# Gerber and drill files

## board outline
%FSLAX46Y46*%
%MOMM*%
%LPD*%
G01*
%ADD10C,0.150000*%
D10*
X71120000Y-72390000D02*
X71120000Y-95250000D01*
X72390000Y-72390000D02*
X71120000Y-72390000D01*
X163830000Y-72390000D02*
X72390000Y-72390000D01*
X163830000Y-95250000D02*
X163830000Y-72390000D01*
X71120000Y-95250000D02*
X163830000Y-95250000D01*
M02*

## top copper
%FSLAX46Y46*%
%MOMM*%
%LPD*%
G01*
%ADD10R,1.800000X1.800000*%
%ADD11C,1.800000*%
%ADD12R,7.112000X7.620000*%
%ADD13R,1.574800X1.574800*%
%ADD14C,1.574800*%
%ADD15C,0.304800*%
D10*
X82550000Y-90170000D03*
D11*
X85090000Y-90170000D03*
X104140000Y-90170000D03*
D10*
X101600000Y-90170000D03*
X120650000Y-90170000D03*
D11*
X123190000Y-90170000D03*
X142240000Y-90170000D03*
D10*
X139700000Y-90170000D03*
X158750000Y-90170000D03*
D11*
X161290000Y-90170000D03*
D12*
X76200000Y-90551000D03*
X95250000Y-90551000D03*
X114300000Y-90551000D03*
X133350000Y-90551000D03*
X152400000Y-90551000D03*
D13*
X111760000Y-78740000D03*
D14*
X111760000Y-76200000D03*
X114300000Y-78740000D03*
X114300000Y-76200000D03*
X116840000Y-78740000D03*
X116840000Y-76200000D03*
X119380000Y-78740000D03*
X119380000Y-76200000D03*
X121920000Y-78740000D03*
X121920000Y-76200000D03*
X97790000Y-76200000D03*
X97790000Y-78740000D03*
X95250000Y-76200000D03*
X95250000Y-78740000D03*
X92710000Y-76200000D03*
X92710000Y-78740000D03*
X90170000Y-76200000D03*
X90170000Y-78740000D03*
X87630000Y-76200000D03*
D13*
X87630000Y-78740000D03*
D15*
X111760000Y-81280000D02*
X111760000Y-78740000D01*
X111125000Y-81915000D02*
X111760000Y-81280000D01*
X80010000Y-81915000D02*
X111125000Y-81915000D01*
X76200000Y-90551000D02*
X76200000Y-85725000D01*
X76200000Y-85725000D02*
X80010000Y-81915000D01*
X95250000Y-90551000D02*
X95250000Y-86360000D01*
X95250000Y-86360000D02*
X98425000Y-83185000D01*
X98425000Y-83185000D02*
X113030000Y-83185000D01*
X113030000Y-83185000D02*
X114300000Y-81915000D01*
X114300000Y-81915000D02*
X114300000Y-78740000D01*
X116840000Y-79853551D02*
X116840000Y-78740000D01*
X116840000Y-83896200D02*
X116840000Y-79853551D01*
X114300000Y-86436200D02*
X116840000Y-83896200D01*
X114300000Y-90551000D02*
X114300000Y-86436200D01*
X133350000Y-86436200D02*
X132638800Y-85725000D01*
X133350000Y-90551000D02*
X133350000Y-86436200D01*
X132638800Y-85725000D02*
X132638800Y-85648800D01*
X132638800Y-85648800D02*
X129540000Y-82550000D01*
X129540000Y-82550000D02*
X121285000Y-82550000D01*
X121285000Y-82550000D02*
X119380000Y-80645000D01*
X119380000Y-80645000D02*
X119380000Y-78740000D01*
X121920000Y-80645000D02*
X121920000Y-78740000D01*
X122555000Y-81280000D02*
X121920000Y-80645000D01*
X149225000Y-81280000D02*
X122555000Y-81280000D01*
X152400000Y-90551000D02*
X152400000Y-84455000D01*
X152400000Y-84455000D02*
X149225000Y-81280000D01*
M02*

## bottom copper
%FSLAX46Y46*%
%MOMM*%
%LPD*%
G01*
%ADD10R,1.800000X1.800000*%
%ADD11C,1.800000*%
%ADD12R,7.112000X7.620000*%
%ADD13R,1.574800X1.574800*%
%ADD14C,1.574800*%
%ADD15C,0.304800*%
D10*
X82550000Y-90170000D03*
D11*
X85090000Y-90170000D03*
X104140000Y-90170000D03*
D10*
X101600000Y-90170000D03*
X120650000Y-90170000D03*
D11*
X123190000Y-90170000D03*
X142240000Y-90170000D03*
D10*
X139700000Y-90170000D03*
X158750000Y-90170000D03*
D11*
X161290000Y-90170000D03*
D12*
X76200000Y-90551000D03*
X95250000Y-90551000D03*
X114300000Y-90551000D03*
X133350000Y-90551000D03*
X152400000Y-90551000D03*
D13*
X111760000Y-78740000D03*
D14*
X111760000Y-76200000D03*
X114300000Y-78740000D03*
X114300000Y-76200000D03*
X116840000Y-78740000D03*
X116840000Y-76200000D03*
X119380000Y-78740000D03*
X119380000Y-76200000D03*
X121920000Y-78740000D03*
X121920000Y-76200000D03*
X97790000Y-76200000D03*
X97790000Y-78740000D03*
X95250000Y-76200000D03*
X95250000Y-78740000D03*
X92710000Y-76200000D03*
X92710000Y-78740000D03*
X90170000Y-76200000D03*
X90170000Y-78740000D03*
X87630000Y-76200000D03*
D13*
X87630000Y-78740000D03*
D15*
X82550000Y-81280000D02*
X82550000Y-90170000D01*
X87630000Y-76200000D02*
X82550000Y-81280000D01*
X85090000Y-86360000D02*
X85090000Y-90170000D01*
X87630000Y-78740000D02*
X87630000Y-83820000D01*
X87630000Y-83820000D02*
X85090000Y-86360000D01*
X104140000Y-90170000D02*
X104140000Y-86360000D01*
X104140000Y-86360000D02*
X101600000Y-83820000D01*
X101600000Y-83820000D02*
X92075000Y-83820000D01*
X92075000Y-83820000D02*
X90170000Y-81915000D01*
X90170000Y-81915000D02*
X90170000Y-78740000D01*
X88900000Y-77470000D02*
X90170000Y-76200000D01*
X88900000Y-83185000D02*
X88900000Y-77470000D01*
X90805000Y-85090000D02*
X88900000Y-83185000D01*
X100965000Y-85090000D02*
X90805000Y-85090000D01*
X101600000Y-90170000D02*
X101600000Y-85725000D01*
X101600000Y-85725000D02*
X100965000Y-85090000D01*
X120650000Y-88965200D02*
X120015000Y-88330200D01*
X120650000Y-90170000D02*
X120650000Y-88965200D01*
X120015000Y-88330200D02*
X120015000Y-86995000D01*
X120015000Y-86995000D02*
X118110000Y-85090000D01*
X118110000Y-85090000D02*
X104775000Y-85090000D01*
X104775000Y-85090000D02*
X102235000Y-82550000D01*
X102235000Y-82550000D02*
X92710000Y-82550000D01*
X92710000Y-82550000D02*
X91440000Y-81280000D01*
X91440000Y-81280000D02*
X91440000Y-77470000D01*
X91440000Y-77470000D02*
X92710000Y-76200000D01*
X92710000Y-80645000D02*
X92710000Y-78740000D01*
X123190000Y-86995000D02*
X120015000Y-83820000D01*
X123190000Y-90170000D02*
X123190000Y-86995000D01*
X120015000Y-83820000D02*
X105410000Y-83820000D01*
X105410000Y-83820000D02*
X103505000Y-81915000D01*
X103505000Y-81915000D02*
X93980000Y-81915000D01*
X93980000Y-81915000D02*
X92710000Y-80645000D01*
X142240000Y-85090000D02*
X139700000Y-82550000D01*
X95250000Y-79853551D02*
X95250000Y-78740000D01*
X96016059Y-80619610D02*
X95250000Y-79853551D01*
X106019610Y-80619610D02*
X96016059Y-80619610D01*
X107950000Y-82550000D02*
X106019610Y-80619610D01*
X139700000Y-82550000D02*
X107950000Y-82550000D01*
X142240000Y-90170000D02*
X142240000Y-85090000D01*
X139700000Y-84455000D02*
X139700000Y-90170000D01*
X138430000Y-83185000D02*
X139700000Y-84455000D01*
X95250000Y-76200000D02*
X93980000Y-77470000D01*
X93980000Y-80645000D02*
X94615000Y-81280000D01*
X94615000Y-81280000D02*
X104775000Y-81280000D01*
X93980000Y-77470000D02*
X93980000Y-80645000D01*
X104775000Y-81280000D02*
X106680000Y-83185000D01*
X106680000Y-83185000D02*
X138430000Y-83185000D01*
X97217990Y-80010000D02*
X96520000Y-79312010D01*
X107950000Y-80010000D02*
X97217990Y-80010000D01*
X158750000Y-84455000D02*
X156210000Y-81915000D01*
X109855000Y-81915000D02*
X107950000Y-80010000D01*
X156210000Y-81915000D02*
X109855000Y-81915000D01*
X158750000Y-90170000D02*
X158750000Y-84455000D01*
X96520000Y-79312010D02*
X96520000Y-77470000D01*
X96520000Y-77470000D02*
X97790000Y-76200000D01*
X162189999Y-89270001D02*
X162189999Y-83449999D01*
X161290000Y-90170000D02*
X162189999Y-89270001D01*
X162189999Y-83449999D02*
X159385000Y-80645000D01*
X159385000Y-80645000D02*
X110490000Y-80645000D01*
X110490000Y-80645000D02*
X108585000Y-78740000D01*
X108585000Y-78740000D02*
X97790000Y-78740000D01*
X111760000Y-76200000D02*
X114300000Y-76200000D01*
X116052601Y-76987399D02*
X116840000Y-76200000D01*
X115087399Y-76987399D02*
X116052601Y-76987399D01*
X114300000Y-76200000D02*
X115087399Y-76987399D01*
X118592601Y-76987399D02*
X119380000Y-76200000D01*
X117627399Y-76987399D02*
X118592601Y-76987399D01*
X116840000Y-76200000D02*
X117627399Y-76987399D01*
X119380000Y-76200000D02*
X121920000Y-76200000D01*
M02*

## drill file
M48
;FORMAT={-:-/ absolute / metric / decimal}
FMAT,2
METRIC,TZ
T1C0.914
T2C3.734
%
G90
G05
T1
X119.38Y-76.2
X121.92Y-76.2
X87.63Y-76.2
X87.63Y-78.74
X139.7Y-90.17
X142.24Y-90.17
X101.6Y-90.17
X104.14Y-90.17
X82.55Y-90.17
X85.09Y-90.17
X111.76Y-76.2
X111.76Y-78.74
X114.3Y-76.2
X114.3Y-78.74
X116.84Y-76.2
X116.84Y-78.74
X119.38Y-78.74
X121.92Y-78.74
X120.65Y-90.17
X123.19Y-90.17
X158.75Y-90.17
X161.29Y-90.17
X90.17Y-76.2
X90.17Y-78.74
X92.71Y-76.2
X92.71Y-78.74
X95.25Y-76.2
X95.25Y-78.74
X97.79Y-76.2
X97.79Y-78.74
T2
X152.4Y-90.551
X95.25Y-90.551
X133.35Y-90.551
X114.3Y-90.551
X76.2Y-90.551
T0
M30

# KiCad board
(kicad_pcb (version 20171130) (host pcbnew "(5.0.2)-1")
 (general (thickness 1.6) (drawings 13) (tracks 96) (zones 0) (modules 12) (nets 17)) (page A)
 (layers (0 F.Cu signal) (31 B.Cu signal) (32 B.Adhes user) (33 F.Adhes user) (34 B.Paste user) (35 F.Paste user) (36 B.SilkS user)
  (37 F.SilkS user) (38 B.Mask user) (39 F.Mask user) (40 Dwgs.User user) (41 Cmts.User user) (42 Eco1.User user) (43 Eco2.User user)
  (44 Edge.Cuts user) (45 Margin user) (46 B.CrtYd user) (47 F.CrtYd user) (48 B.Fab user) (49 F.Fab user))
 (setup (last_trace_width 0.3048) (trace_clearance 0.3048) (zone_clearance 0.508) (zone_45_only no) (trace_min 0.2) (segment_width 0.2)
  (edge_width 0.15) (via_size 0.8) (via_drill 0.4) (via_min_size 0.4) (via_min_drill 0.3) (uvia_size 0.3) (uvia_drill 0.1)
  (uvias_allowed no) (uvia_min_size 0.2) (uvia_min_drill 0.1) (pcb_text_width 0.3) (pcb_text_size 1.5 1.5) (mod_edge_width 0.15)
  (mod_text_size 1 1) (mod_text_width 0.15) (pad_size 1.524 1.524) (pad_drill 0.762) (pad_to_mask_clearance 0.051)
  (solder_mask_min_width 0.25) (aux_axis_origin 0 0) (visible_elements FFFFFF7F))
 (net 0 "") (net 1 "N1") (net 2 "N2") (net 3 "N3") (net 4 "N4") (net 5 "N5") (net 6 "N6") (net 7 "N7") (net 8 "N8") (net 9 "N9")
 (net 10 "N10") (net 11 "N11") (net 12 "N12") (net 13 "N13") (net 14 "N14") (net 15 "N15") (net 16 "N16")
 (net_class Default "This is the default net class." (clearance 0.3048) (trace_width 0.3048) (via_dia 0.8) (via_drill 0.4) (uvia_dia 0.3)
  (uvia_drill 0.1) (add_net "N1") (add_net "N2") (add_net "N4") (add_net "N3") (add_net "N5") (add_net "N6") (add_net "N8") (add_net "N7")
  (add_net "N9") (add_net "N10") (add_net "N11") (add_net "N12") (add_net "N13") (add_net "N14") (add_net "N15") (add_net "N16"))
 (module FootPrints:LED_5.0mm (layer F.Cu) (at 82.55 90.17)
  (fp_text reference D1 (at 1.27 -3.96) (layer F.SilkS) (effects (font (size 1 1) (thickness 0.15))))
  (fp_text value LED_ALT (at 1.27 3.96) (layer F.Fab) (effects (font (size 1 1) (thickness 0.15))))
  (pad 1 thru_hole rect (at 0 0) (size 1.8 1.8) (drill 0.9144) (layers *.Cu *.Mask) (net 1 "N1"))
  (pad 2 thru_hole circle (at 2.54 0) (size 1.8 1.8) (drill 0.9144) (layers *.Cu *.Mask) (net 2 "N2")))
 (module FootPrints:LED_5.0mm (layer F.Cu) (at 101.6 90.17)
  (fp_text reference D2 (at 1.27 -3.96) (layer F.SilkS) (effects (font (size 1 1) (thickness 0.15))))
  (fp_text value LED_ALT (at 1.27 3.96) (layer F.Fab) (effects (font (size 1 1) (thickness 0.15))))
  (pad 2 thru_hole circle (at 2.54 0) (size 1.8 1.8) (drill 0.9144) (layers *.Cu *.Mask) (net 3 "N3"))
  (pad 1 thru_hole rect (at 0 0) (size 1.8 1.8) (drill 0.9144) (layers *.Cu *.Mask) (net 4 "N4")))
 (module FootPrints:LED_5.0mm (layer F.Cu) (at 120.65 90.17)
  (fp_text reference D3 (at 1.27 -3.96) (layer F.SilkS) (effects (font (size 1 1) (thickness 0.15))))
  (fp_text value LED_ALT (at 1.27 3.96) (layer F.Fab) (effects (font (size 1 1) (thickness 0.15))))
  (pad 1 thru_hole rect (at 0 0) (size 1.8 1.8) (drill 0.9144) (layers *.Cu *.Mask) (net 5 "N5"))
  (pad 2 thru_hole circle (at 2.54 0) (size 1.8 1.8) (drill 0.9144) (layers *.Cu *.Mask) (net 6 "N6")))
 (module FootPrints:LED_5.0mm (layer F.Cu) (at 139.7 90.17)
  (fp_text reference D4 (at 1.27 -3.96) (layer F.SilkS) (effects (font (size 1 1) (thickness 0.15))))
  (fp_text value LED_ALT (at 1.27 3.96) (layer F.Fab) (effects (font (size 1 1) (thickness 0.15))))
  (pad 2 thru_hole circle (at 2.54 0) (size 1.8 1.8) (drill 0.9144) (layers *.Cu *.Mask) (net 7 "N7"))
  (pad 1 thru_hole rect (at 0 0) (size 1.8 1.8) (drill 0.9144) (layers *.Cu *.Mask) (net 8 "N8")))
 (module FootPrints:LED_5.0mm (layer F.Cu) (at 158.75 90.17)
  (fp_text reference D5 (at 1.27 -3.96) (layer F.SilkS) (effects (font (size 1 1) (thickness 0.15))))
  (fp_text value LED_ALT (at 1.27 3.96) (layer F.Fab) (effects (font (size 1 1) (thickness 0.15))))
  (pad 1 thru_hole rect (at 0 0) (size 1.8 1.8) (drill 0.9144) (layers *.Cu *.Mask) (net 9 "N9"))
  (pad 2 thru_hole circle (at 2.54 0) (size 1.8 1.8) (drill 0.9144) (layers *.Cu *.Mask) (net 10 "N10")))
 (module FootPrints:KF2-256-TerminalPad (layer F.Cu) (at 76.2 95.25)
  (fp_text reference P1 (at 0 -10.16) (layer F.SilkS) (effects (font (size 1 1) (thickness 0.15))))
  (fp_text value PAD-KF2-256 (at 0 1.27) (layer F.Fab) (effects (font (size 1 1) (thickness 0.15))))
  (pad 1 thru_hole rect (at 0 -4.699) (size 7.112 7.62) (drill 3.7338) (layers *.Cu *.Mask F.SilkS) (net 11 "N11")))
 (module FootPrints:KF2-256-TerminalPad (layer F.Cu) (at 95.25 95.25)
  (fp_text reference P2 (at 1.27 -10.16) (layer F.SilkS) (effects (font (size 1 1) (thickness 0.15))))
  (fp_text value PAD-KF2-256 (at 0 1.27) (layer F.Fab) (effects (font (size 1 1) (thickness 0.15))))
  (pad 1 thru_hole rect (at 0 -4.699) (size 7.112 7.62) (drill 3.7338) (layers *.Cu *.Mask F.SilkS) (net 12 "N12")))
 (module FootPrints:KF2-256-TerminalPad (layer F.Cu) (at 114.3 95.25)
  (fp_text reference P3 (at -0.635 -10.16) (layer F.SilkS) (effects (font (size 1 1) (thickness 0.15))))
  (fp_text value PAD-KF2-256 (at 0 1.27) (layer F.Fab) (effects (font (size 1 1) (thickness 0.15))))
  (pad 1 thru_hole rect (at 0 -4.699) (size 7.112 7.62) (drill 3.7338) (layers *.Cu *.Mask F.SilkS) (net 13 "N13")))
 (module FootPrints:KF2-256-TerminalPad (layer F.Cu) (at 133.35 95.25)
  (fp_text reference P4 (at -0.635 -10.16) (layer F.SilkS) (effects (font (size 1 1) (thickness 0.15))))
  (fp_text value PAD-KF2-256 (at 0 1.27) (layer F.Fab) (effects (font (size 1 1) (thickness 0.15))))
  (pad 1 thru_hole rect (at 0 -4.699) (size 7.112 7.62) (drill 3.7338) (layers *.Cu *.Mask F.SilkS) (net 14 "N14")))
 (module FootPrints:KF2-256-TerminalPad (layer F.Cu) (at 152.4 95.25)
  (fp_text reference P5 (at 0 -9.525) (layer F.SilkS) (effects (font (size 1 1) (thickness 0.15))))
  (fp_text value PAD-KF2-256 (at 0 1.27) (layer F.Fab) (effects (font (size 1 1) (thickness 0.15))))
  (pad 1 thru_hole rect (at 0 -4.699) (size 7.112 7.62) (drill 3.7338) (layers *.Cu *.Mask F.SilkS) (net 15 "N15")))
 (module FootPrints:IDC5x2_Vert (layer F.Cu) (at 116.84 77.47 180)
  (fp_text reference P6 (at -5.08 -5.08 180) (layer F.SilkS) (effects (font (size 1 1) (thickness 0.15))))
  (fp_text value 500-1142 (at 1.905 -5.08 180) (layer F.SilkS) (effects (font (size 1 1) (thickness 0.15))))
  (pad 1 thru_hole rect (at 5.08 -1.27 180) (size 1.5748 1.5748) (drill 0.9144) (layers *.Cu *.Mask F.SilkS) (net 11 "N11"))
  (pad 2 thru_hole circle (at 5.08 1.27 180) (size 1.5748 1.5748) (drill 0.9144) (layers *.Cu *.Mask F.SilkS) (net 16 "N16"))
  (pad 3 thru_hole circle (at 2.54 -1.27 180) (size 1.5748 1.5748) (drill 0.9144) (layers *.Cu *.Mask F.SilkS) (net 12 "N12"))
  (pad 4 thru_hole circle (at 2.54 1.27 180) (size 1.5748 1.5748) (drill 0.9144) (layers *.Cu *.Mask F.SilkS) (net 16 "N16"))
  (pad 5 thru_hole circle (at 0 -1.27 180) (size 1.5748 1.5748) (drill 0.9144) (layers *.Cu *.Mask F.SilkS) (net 13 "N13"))
  (pad 6 thru_hole circle (at 0 1.27 180) (size 1.5748 1.5748) (drill 0.9144) (layers *.Cu *.Mask F.SilkS) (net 16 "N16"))
  (pad 7 thru_hole circle (at -2.54 -1.27 180) (size 1.5748 1.5748) (drill 0.9144) (layers *.Cu *.Mask F.SilkS) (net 14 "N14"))
  (pad 8 thru_hole circle (at -2.54 1.27 180) (size 1.5748 1.5748) (drill 0.9144) (layers *.Cu *.Mask F.SilkS) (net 16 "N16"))
  (pad 9 thru_hole circle (at -5.08 -1.27 180) (size 1.5748 1.5748) (drill 0.9144) (layers *.Cu *.Mask F.SilkS) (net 15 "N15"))
  (pad 10 thru_hole circle (at -5.08 1.27 180) (size 1.5748 1.5748) (drill 0.9144) (layers *.Cu *.Mask F.SilkS) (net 16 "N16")))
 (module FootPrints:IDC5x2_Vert (layer F.Cu) (at 92.71 77.47 180)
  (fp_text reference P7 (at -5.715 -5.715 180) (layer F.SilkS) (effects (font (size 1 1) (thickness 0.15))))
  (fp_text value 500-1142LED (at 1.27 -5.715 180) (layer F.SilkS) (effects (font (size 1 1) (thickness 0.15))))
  (pad 10 thru_hole circle (at -5.08 1.27 180) (size 1.5748 1.5748) (drill 0.9144) (layers *.Cu *.Mask F.SilkS) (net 9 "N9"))
  (pad 9 thru_hole circle (at -5.08 -1.27 180) (size 1.5748 1.5748) (drill 0.9144) (layers *.Cu *.Mask F.SilkS) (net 10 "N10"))
  (pad 8 thru_hole circle (at -2.54 1.27 180) (size 1.5748 1.5748) (drill 0.9144) (layers *.Cu *.Mask F.SilkS) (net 8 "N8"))
  (pad 7 thru_hole circle (at -2.54 -1.27 180) (size 1.5748 1.5748) (drill 0.9144) (layers *.Cu *.Mask F.SilkS) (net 7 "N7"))
  (pad 6 thru_hole circle (at 0 1.27 180) (size 1.5748 1.5748) (drill 0.9144) (layers *.Cu *.Mask F.SilkS) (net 5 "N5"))
  (pad 5 thru_hole circle (at 0 -1.27 180) (size 1.5748 1.5748) (drill 0.9144) (layers *.Cu *.Mask F.SilkS) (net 6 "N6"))
  (pad 4 thru_hole circle (at 2.54 1.27 180) (size 1.5748 1.5748) (drill 0.9144) (layers *.Cu *.Mask F.SilkS) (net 4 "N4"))
  (pad 3 thru_hole circle (at 2.54 -1.27 180) (size 1.5748 1.5748) (drill 0.9144) (layers *.Cu *.Mask F.SilkS) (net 3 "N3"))
  (pad 2 thru_hole circle (at 5.08 1.27 180) (size 1.5748 1.5748) (drill 0.9144) (layers *.Cu *.Mask F.SilkS) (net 1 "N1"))
  (pad 1 thru_hole rect (at 5.08 -1.27 180) (size 1.5748 1.5748) (drill 0.9144) (layers *.Cu *.Mask F.SilkS) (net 2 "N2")))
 (gr_line (start 71.12 72.39) (end 71.12 95.25) (layer Edge.Cuts) (width 0.15))
 (gr_line (start 72.39 72.39) (end 71.12 72.39) (layer Edge.Cuts) (width 0.15))
 (gr_line (start 163.83 72.39) (end 72.39 72.39) (layer Edge.Cuts) (width 0.15))
 (gr_line (start 163.83 95.25) (end 163.83 72.39) (layer Edge.Cuts) (width 0.15))
 (gr_line (start 71.12 95.25) (end 163.83 95.25) (layer Edge.Cuts) (width 0.15))
 (segment (start 82.55 81.28) (end 82.55 90.17) (width 0.3048) (layer B.Cu) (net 1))
 (segment (start 87.63 76.2) (end 82.55 81.28) (width 0.3048) (layer B.Cu) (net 1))
 (segment (start 85.09 86.36) (end 85.09 90.17) (width 0.3048) (layer B.Cu) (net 2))
 (segment (start 87.63 78.74) (end 87.63 83.82) (width 0.3048) (layer B.Cu) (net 2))
 (segment (start 87.63 83.82) (end 85.09 86.36) (width 0.3048) (layer B.Cu) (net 2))
 (segment (start 104.14 90.17) (end 104.14 86.36) (width 0.3048) (layer B.Cu) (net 3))
 (segment (start 104.14 86.36) (end 101.6 83.82) (width 0.3048) (layer B.Cu) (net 3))
 (segment (start 101.6 83.82) (end 92.075 83.82) (width 0.3048) (layer B.Cu) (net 3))
 (segment (start 92.075 83.82) (end 90.17 81.915) (width 0.3048) (layer B.Cu) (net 3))
 (segment (start 90.17 81.915) (end 90.17 78.74) (width 0.3048) (layer B.Cu) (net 3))
 (segment (start 88.9 77.47) (end 90.17 76.2) (width 0.3048) (layer B.Cu) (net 4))
 (segment (start 88.9 83.185) (end 88.9 77.47) (width 0.3048) (layer B.Cu) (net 4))
 (segment (start 90.805 85.09) (end 88.9 83.185) (width 0.3048) (layer B.Cu) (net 4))
 (segment (start 100.965 85.09) (end 90.805 85.09) (width 0.3048) (layer B.Cu) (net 4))
 (segment (start 101.6 90.17) (end 101.6 85.725) (width 0.3048) (layer B.Cu) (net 4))
 (segment (start 101.6 85.725) (end 100.965 85.09) (width 0.3048) (layer B.Cu) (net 4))
 (segment (start 120.65 88.9652) (end 120.015 88.3302) (width 0.3048) (layer B.Cu) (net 5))
 (segment (start 120.65 90.17) (end 120.65 88.9652) (width 0.3048) (layer B.Cu) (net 5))
 (segment (start 120.015 88.3302) (end 120.015 86.995) (width 0.3048) (layer B.Cu) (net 5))
 (segment (start 120.015 86.995) (end 118.11 85.09) (width 0.3048) (layer B.Cu) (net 5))
 (segment (start 118.11 85.09) (end 104.775 85.09) (width 0.3048) (layer B.Cu) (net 5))
 (segment (start 104.775 85.09) (end 102.235 82.55) (width 0.3048) (layer B.Cu) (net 5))
 (segment (start 102.235 82.55) (end 92.71 82.55) (width 0.3048) (layer B.Cu) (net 5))
 (segment (start 92.71 82.55) (end 91.44 81.28) (width 0.3048) (layer B.Cu) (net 5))
 (segment (start 91.44 81.28) (end 91.44 77.47) (width 0.3048) (layer B.Cu) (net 5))
 (segment (start 91.44 77.47) (end 92.71 76.2) (width 0.3048) (layer B.Cu) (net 5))
 (segment (start 92.71 80.645) (end 92.71 78.74) (width 0.3048) (layer B.Cu) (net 6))
 (segment (start 123.19 86.995) (end 120.015 83.82) (width 0.3048) (layer B.Cu) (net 6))
 (segment (start 123.19 90.17) (end 123.19 86.995) (width 0.3048) (layer B.Cu) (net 6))
 (segment (start 120.015 83.82) (end 105.41 83.82) (width 0.3048) (layer B.Cu) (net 6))
 (segment (start 105.41 83.82) (end 103.505 81.915) (width 0.3048) (layer B.Cu) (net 6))
 (segment (start 103.505 81.915) (end 93.98 81.915) (width 0.3048) (layer B.Cu) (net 6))
 (segment (start 93.98 81.915) (end 92.71 80.645) (width 0.3048) (layer B.Cu) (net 6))
 (segment (start 142.24 85.09) (end 139.7 82.55) (width 0.3048) (layer B.Cu) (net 7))
 (segment (start 95.25 79.853551) (end 95.25 78.74) (width 0.3048) (layer B.Cu) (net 7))
 (segment (start 96.016059 80.61961) (end 95.25 79.853551) (width 0.3048) (layer B.Cu) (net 7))
 (segment (start 106.01961 80.61961) (end 96.016059 80.61961) (width 0.3048) (layer B.Cu) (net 7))
 (segment (start 107.95 82.55) (end 106.01961 80.61961) (width 0.3048) (layer B.Cu) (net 7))
 (segment (start 139.7 82.55) (end 107.95 82.55) (width 0.3048) (layer B.Cu) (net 7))
 (segment (start 142.24 90.17) (end 142.24 85.09) (width 0.3048) (layer B.Cu) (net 7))
 (segment (start 139.7 84.455) (end 139.7 90.17) (width 0.3048) (layer B.Cu) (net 8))
 (segment (start 138.43 83.185) (end 139.7 84.455) (width 0.3048) (layer B.Cu) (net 8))
 (segment (start 95.25 76.2) (end 93.98 77.47) (width 0.3048) (layer B.Cu) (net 8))
 (segment (start 93.98 80.645) (end 94.615 81.28) (width 0.3048) (layer B.Cu) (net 8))
 (segment (start 94.615 81.28) (end 104.775 81.28) (width 0.3048) (layer B.Cu) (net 8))
 (segment (start 93.98 77.47) (end 93.98 80.645) (width 0.3048) (layer B.Cu) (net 8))
 (segment (start 104.775 81.28) (end 106.68 83.185) (width 0.3048) (layer B.Cu) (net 8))
 (segment (start 106.68 83.185) (end 138.43 83.185) (width 0.3048) (layer B.Cu) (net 8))
 (segment (start 97.21799 80.01) (end 96.52 79.31201) (width 0.3048) (layer B.Cu) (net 9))
 (segment (start 107.95 80.01) (end 97.21799 80.01) (width 0.3048) (layer B.Cu) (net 9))
 (segment (start 158.75 84.455) (end 156.21 81.915) (width 0.3048) (layer B.Cu) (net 9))
 (segment (start 109.855 81.915) (end 107.95 80.01) (width 0.3048) (layer B.Cu) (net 9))
 (segment (start 156.21 81.915) (end 109.855 81.915) (width 0.3048) (layer B.Cu) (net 9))
 (segment (start 158.75 90.17) (end 158.75 84.455) (width 0.3048) (layer B.Cu) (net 9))
 (segment (start 96.52 79.31201) (end 96.52 77.47) (width 0.3048) (layer B.Cu) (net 9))
 (segment (start 96.52 77.47) (end 97.79 76.2) (width 0.3048) (layer B.Cu) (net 9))
 (segment (start 162.189999 89.270001) (end 162.189999 83.449999) (width 0.3048) (layer B.Cu) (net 10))
 (segment (start 161.29 90.17) (end 162.189999 89.270001) (width 0.3048) (layer B.Cu) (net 10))
 (segment (start 162.189999 83.449999) (end 159.385 80.645) (width 0.3048) (layer B.Cu) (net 10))
 (segment (start 159.385 80.645) (end 110.49 80.645) (width 0.3048) (layer B.Cu) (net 10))
 (segment (start 110.49 80.645) (end 108.585 78.74) (width 0.3048) (layer B.Cu) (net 10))
 (segment (start 108.585 78.74) (end 97.79 78.74) (width 0.3048) (layer B.Cu) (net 10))
 (segment (start 111.76 81.28) (end 111.76 78.74) (width 0.3048) (layer F.Cu) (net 11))
 (segment (start 111.125 81.915) (end 111.76 81.28) (width 0.3048) (layer F.Cu) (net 11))
 (segment (start 80.01 81.915) (end 111.125 81.915) (width 0.3048) (layer F.Cu) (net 11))
 (segment (start 76.2 90.551) (end 76.2 85.725) (width 0.3048) (layer F.Cu) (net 11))
 (segment (start 76.2 85.725) (end 80.01 81.915) (width 0.3048) (layer F.Cu) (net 11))
 (segment (start 95.25 90.551) (end 95.25 86.36) (width 0.3048) (layer F.Cu) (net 12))
 (segment (start 95.25 86.36) (end 98.425 83.185) (width 0.3048) (layer F.Cu) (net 12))
 (segment (start 98.425 83.185) (end 113.03 83.185) (width 0.3048) (layer F.Cu) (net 12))
 (segment (start 113.03 83.185) (end 114.3 81.915) (width 0.3048) (layer F.Cu) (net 12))
 (segment (start 114.3 81.915) (end 114.3 78.74) (width 0.3048) (layer F.Cu) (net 12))
 (segment (start 116.84 79.853551) (end 116.84 78.74) (width 0.3048) (layer F.Cu) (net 13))
 (segment (start 116.84 83.8962) (end 116.84 79.853551) (width 0.3048) (layer F.Cu) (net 13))
 (segment (start 114.3 86.4362) (end 116.84 83.8962) (width 0.3048) (layer F.Cu) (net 13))
 (segment (start 114.3 90.551) (end 114.3 86.4362) (width 0.3048) (layer F.Cu) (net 13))
 (segment (start 133.35 86.4362) (end 132.6388 85.725) (width 0.3048) (layer F.Cu) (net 14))
 (segment (start 133.35 90.551) (end 133.35 86.4362) (width 0.3048) (layer F.Cu) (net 14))
 (segment (start 132.6388 85.725) (end 132.6388 85.6488) (width 0.3048) (layer F.Cu) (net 14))
 (segment (start 132.6388 85.6488) (end 129.54 82.55) (width 0.3048) (layer F.Cu) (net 14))
 (segment (start 129.54 82.55) (end 121.285 82.55) (width 0.3048) (layer F.Cu) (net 14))
 (segment (start 121.285 82.55) (end 119.38 80.645) (width 0.3048) (layer F.Cu) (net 14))
 (segment (start 119.38 80.645) (end 119.38 78.74) (width 0.3048) (layer F.Cu) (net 14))
 (segment (start 121.92 80.645) (end 121.92 78.74) (width 0.3048) (layer F.Cu) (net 15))
 (segment (start 122.555 81.28) (end 121.92 80.645) (width 0.3048) (layer F.Cu) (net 15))
 (segment (start 149.225 81.28) (end 122.555 81.28) (width 0.3048) (layer F.Cu) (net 15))
 (segment (start 152.4 90.551) (end 152.4 84.455) (width 0.3048) (layer F.Cu) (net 15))
 (segment (start 152.4 84.455) (end 149.225 81.28) (width 0.3048) (layer F.Cu) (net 15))
 (segment (start 111.76 76.2) (end 114.3 76.2) (width 0.3048) (layer B.Cu) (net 16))
 (segment (start 116.052601 76.987399) (end 116.84 76.2) (width 0.3048) (layer B.Cu) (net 16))
 (segment (start 115.087399 76.987399) (end 116.052601 76.987399) (width 0.3048) (layer B.Cu) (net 16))
 (segment (start 114.3 76.2) (end 115.087399 76.987399) (width 0.3048) (layer B.Cu) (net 16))
 (segment (start 118.592601 76.987399) (end 119.38 76.2) (width 0.3048) (layer B.Cu) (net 16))
 (segment (start 117.627399 76.987399) (end 118.592601 76.987399) (width 0.3048) (layer B.Cu) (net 16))
 (segment (start 116.84 76.2) (end 117.627399 76.987399) (width 0.3048) (layer B.Cu) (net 16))
 (segment (start 119.38 76.2) (end 121.92 76.2) (width 0.3048) (layer B.Cu) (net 16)))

